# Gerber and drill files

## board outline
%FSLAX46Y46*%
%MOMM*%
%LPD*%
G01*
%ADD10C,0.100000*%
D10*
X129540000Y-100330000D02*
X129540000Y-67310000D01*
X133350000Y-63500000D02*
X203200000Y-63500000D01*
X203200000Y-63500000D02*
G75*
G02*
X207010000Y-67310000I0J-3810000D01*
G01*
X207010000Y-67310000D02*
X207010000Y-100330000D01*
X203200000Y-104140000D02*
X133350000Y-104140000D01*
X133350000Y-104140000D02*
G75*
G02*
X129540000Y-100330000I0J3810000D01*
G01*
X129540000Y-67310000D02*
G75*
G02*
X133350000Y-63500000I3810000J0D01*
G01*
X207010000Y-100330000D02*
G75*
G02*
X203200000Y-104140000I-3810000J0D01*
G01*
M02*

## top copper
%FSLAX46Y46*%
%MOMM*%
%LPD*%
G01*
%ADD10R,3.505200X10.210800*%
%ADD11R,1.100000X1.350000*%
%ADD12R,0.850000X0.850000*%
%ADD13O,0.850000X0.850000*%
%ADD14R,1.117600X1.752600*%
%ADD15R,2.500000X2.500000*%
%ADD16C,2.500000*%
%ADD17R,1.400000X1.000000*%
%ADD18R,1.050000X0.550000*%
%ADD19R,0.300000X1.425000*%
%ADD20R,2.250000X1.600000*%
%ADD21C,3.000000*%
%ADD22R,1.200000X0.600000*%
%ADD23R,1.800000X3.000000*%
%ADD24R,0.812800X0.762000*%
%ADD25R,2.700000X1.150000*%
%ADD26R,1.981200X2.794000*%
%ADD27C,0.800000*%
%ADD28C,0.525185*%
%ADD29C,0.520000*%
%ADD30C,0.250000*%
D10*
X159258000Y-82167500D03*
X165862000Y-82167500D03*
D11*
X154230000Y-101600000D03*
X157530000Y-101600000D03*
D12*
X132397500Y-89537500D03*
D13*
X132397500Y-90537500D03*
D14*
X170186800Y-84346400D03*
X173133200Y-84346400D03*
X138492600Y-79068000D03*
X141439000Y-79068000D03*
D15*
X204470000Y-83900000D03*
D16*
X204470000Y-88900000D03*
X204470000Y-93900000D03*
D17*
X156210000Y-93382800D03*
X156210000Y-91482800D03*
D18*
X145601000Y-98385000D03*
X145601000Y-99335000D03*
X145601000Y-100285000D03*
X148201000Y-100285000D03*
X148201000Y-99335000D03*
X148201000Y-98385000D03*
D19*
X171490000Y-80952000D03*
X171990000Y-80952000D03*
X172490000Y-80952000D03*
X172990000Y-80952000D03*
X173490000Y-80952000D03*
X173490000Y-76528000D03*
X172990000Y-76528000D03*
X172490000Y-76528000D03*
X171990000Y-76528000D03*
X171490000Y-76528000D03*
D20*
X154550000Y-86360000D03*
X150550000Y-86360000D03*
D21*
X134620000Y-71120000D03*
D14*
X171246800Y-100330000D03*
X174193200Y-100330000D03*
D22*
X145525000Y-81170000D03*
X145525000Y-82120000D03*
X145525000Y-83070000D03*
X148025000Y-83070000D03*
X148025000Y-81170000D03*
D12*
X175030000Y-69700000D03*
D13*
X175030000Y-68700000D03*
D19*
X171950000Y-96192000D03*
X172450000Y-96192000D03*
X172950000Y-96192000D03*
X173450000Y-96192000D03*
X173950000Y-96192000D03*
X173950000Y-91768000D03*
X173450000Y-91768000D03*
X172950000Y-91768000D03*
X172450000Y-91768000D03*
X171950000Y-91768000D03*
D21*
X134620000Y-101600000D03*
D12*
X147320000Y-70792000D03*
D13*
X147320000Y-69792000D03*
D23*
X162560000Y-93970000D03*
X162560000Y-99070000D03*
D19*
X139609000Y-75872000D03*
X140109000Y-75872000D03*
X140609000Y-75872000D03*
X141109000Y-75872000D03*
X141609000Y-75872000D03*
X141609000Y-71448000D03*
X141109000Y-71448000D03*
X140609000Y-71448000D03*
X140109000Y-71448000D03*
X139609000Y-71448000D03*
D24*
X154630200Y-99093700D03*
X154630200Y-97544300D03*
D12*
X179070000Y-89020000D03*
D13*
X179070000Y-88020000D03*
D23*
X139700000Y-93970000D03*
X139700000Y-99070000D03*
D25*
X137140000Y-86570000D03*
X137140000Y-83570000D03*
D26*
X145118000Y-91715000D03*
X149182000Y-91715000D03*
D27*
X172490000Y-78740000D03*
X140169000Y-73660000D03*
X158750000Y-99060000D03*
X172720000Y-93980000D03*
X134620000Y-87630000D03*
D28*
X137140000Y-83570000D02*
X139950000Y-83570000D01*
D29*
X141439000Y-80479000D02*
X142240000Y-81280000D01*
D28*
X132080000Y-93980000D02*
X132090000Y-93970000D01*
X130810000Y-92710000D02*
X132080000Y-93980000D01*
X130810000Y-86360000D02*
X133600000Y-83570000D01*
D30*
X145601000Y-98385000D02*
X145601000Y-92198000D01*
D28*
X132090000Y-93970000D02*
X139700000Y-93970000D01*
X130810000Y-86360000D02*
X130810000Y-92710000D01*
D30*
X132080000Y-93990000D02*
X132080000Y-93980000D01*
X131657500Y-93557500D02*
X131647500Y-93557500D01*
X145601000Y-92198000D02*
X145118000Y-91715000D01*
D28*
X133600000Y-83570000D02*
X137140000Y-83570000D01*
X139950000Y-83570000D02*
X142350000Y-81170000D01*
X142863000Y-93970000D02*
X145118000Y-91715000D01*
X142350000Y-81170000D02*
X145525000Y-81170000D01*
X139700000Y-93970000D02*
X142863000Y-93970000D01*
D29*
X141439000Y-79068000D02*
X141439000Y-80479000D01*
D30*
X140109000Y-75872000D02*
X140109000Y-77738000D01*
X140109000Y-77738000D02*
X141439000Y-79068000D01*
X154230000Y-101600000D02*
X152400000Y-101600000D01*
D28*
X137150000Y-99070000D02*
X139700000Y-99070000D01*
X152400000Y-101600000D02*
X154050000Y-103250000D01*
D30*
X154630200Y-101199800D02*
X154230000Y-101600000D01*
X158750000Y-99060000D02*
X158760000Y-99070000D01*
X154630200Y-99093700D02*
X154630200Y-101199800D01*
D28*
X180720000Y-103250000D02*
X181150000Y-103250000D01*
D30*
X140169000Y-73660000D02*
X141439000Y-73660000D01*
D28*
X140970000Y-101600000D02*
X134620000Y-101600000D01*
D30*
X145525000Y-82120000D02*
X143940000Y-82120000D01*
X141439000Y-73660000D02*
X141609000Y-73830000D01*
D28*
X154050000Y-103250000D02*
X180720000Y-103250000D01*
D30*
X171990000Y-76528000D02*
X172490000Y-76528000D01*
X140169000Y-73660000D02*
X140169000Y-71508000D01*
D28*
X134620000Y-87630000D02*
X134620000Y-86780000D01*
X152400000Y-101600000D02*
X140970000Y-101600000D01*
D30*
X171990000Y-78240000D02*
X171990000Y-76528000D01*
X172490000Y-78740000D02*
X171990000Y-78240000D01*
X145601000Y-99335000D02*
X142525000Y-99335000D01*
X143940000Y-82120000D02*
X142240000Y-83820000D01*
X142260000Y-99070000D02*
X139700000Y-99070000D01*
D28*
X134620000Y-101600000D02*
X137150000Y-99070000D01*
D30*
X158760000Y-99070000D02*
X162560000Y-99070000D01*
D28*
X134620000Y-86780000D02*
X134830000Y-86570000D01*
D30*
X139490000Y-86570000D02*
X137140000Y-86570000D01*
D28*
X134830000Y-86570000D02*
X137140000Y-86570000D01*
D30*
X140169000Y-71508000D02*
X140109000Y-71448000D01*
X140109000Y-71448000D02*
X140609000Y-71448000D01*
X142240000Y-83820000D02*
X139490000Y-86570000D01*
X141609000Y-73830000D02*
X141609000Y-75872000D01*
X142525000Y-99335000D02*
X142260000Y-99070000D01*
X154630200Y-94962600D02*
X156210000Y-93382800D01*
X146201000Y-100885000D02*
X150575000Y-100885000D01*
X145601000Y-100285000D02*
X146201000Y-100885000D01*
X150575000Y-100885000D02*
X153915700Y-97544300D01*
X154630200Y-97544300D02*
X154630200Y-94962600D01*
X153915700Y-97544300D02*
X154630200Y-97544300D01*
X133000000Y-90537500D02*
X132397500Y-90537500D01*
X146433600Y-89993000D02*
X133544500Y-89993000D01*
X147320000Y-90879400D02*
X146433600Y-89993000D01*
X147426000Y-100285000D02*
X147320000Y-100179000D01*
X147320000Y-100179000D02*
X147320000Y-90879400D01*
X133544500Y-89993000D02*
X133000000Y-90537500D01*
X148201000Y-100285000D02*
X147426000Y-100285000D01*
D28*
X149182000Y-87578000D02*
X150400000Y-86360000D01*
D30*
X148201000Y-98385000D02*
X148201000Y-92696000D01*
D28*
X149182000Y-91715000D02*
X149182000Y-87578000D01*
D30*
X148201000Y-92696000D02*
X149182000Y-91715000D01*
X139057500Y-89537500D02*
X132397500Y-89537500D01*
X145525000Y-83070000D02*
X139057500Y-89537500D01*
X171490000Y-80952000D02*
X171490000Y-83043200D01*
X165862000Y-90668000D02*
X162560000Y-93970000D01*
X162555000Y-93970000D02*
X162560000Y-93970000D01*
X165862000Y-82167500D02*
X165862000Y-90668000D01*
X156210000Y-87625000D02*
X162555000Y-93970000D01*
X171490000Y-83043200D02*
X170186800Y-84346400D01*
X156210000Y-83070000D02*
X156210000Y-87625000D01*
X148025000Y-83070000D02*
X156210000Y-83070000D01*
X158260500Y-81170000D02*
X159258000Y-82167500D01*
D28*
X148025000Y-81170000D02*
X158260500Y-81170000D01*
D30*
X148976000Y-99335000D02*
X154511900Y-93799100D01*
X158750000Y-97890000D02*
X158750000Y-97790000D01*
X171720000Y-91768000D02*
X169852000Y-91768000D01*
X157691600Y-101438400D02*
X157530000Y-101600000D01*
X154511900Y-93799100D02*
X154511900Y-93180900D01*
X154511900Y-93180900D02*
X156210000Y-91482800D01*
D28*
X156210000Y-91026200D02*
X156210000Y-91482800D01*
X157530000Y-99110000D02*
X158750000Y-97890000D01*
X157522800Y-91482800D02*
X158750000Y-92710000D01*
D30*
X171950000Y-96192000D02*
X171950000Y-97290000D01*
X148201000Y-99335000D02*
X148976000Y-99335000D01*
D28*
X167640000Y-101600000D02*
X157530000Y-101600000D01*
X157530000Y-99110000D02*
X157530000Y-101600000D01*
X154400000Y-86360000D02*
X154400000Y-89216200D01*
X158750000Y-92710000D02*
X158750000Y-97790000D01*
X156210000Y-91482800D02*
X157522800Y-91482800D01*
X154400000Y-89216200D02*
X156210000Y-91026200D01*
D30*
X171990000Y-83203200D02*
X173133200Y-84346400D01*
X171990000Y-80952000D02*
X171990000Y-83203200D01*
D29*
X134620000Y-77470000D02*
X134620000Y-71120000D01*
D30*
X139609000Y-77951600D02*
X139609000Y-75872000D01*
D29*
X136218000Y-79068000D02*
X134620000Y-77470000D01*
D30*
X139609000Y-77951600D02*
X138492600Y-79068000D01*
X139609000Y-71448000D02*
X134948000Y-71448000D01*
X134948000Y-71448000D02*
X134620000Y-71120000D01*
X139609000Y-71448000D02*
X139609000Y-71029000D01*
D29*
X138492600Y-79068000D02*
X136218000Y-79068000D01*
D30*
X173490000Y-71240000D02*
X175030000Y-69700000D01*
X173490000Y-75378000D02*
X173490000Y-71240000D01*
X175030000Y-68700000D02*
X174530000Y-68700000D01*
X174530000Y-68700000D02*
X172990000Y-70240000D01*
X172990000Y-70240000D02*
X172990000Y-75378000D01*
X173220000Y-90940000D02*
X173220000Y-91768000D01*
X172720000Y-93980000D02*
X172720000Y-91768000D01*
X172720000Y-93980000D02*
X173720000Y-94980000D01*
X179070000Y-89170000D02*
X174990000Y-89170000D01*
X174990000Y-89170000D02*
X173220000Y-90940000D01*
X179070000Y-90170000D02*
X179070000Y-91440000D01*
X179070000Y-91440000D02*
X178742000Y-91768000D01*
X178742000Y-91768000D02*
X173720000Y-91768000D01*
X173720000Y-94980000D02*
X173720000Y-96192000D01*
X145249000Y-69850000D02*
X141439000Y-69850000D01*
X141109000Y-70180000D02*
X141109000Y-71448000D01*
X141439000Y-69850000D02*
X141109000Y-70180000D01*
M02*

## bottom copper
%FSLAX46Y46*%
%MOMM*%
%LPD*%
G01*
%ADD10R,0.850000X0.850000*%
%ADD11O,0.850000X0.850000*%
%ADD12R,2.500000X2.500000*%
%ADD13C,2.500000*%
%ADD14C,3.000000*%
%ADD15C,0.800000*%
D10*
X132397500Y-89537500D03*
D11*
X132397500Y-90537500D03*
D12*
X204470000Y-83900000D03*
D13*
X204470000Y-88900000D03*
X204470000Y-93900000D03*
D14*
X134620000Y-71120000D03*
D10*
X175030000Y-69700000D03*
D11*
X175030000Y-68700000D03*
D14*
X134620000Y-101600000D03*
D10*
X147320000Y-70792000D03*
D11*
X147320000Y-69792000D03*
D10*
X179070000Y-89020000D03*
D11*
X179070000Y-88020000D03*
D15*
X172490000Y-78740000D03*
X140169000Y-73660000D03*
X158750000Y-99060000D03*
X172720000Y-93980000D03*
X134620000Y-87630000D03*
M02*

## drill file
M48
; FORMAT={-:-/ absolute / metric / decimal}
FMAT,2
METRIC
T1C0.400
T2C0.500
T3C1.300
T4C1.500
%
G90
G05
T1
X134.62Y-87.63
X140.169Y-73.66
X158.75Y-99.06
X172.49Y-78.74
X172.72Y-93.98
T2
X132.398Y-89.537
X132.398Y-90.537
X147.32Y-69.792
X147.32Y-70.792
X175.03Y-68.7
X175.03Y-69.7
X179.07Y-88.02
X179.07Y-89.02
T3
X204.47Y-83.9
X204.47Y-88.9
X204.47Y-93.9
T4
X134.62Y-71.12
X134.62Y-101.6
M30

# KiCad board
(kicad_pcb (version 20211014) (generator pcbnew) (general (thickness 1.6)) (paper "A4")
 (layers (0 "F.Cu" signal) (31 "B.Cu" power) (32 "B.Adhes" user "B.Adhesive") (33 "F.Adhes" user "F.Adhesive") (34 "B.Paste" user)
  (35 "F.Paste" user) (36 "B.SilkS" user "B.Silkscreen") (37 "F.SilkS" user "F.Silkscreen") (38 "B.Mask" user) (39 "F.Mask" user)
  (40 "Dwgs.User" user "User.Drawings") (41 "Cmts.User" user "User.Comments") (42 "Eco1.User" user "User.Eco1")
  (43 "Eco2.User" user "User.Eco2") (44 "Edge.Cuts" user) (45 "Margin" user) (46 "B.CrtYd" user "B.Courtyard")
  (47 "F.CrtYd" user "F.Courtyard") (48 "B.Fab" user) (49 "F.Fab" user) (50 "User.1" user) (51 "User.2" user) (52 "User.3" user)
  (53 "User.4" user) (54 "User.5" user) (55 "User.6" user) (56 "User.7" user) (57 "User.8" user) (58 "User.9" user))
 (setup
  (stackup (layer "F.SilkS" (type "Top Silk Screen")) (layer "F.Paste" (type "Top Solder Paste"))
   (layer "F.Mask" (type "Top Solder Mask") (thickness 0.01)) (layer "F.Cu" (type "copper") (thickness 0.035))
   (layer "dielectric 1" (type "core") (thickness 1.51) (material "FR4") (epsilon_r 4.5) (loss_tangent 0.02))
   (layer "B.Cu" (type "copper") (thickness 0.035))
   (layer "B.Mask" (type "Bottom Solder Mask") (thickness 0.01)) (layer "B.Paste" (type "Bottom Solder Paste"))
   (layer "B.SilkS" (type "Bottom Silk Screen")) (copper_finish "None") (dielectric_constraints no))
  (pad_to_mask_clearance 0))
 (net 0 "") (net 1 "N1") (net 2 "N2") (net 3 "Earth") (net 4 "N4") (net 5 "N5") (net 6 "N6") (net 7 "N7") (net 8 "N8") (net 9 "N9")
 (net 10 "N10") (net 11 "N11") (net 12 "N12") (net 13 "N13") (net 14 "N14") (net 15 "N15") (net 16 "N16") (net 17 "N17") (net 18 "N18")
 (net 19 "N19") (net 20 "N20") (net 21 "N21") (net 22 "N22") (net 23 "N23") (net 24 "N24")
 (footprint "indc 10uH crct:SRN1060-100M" (layer "F.Cu") (at 162.56 82.1675)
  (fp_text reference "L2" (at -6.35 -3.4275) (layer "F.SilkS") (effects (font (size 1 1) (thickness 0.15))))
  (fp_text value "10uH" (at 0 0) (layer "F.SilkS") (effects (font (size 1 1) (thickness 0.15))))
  (pad "1" smd rect (at -3.302 0) (size 3.5052 10.2108) (layers "F.Cu" "F.Paste" "F.Mask") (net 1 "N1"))
  (pad "2" smd rect (at 3.302 0) (size 3.5052 10.2108) (layers "F.Cu" "F.Paste" "F.Mask") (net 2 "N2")))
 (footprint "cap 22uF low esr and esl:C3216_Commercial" (layer "F.Cu") (at 155.88 101.6)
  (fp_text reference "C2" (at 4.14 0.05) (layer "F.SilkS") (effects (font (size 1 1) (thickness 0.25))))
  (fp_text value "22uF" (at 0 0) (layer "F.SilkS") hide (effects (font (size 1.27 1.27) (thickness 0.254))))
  (pad "1" smd rect (at -1.65 0) (size 1.1 1.35) (layers "F.Cu" "F.Paste" "F.Mask") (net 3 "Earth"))
  (pad "2" smd rect (at 1.65 0) (size 1.1 1.35) (layers "F.Cu" "F.Paste" "F.Mask") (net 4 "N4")))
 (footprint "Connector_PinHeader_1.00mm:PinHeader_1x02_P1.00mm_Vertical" (layer "F.Cu") (at 132.3975 89.5375)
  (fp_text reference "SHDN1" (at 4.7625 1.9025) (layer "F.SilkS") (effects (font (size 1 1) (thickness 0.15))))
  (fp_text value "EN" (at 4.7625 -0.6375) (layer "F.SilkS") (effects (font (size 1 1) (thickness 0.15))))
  (pad "1" thru_hole rect (at 0 0) (size 0.85 0.85) (drill 0.5) (layers *.Cu *.Mask) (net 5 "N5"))
  (pad "2" thru_hole oval (at 0 1) (size 0.85 0.85) (drill 0.5) (layers *.Cu *.Mask) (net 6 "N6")))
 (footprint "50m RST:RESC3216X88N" (layer "F.Cu") (at 171.66 84.3464)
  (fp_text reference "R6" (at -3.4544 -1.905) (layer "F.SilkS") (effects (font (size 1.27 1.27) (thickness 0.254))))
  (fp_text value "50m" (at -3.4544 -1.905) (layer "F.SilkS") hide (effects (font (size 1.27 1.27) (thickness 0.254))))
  (pad "1" smd rect (at -1.4732 0) (size 1.1176 1.7526) (layers "F.Cu" "F.Paste" "F.Mask") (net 2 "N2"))
  (pad "2" smd rect (at 1.4732 0) (size 1.1176 1.7526) (layers "F.Cu" "F.Paste" "F.Mask") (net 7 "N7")))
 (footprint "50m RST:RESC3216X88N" (layer "F.Cu") (at 139.9658 79.068)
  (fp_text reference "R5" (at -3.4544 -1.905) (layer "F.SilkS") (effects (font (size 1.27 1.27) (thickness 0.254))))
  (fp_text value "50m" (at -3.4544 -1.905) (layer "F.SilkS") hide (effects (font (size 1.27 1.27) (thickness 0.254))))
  (pad "1" smd rect (at -1.4732 0) (size 1.1176 1.7526) (layers "F.Cu" "F.Paste" "F.Mask") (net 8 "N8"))
  (pad "2" smd rect (at 1.4732 0) (size 1.1176 1.7526) (layers "F.Cu" "F.Paste" "F.Mask") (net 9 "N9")))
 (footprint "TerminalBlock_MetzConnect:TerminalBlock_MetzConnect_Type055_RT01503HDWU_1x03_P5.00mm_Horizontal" (layer "F.Cu")
  (at 204.47 83.9 -90)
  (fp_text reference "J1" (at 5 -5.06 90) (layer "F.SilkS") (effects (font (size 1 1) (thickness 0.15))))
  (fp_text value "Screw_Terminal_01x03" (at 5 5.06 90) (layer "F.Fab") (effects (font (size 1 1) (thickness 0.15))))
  (pad "1" thru_hole rect (at 0 0 270) (size 2.5 2.5) (drill 1.3) (layers *.Cu *.Mask) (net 7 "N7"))
  (pad "2" thru_hole circle (at 5 0 270) (size 2.5 2.5) (drill 1.3) (layers *.Cu *.Mask) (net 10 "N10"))
  (pad "3" thru_hole circle (at 10 0 270) (size 2.5 2.5) (drill 1.3) (layers *.Cu *.Mask) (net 3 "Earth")))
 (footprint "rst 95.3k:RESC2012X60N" (layer "F.Cu") (at 156.21 92.4328 90)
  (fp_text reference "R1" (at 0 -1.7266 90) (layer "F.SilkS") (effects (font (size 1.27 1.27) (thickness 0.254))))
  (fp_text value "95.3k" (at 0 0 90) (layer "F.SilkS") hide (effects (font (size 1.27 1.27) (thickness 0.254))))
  (pad "1" smd rect (at -0.95 0 90) (size 1 1.4) (layers "F.Cu" "F.Paste" "F.Mask") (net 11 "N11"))
  (pad "2" smd rect (at 0.95 0 90) (size 1 1.4) (layers "F.Cu" "F.Paste" "F.Mask") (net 4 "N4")))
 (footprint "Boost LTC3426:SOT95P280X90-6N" (layer "F.Cu") (at 146.901 99.335)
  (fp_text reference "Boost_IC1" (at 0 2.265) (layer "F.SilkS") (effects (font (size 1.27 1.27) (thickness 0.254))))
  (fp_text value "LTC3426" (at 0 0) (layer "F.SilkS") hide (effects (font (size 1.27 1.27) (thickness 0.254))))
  (pad "1" smd rect (at -1.3 -0.95 90) (size 0.55 1.05) (layers "F.Cu" "F.Paste" "F.Mask") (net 9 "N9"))
  (pad "2" smd rect (at -1.3 0 90) (size 0.55 1.05) (layers "F.Cu" "F.Paste" "F.Mask") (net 3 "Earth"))
  (pad "3" smd rect (at -1.3 0.95 90) (size 0.55 1.05) (layers "F.Cu" "F.Paste" "F.Mask") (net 11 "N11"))
  (pad "4" smd rect (at 1.3 0.95 90) (size 0.55 1.05) (layers "F.Cu" "F.Paste" "F.Mask") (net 6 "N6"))
  (pad "5" smd rect (at 1.3 0 90) (size 0.55 1.05) (layers "F.Cu" "F.Paste" "F.Mask") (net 4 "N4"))
  (pad "6" smd rect (at 1.3 -0.95 90) (size 0.55 1.05) (layers "F.Cu" "F.Paste" "F.Mask") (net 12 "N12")))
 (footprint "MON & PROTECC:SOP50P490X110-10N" (layer "F.Cu") (at 172.49 78.74 90)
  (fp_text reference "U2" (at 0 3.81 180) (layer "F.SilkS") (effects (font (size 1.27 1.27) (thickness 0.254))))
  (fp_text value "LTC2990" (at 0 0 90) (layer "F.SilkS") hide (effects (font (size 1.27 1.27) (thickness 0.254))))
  (pad "1" smd rect (at -2.212 -1 180) (size 0.3 1.425) (layers "F.Cu" "F.Paste" "F.Mask") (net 2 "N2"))
  (pad "2" smd rect (at -2.212 -0.5 180) (size 0.3 1.425) (layers "F.Cu" "F.Paste" "F.Mask") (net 7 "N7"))
  (pad "3" smd rect (at -2.212 0 180) (size 0.3 1.425) (layers "F.Cu" "F.Paste" "F.Mask") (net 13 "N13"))
  (pad "4" smd rect (at -2.212 0.5 180) (size 0.3 1.425) (layers "F.Cu" "F.Paste" "F.Mask") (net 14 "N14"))
  (pad "5" smd rect (at -2.212 1 180) (size 0.3 1.425) (layers "F.Cu" "F.Paste" "F.Mask") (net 3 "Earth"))
  (pad "6" smd rect (at 2.212 1 180) (size 0.3 1.425) (layers "F.Cu" "F.Paste" "F.Mask") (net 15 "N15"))
  (pad "7" smd rect (at 2.212 0.5 180) (size 0.3 1.425) (layers "F.Cu" "F.Paste" "F.Mask") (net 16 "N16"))
  (pad "8" smd rect (at 2.212 0 180) (size 0.3 1.425) (layers "F.Cu" "F.Paste" "F.Mask") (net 3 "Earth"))
  (pad "9" smd rect (at 2.212 -0.5 180) (size 0.3 1.425) (layers "F.Cu" "F.Paste" "F.Mask") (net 3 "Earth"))
  (pad "10" smd rect (at 2.212 -1 180) (size 0.3 1.425) (layers "F.Cu" "F.Paste" "F.Mask") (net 2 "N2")))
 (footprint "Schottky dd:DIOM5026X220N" (layer "F.Cu") (at 152.55 86.36 180)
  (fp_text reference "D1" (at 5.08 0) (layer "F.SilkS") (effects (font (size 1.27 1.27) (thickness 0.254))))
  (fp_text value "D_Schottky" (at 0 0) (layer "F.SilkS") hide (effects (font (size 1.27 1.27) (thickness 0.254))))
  (pad "1" smd rect (at -2 0 270) (size 1.6 2.25) (layers "F.Cu" "F.Paste" "F.Mask") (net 4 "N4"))
  (pad "2" smd rect (at 2 0 270) (size 1.6 2.25) (layers "F.Cu" "F.Paste" "F.Mask") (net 12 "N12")))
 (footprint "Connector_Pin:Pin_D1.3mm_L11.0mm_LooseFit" (layer "F.Cu") (at 134.62 71.12)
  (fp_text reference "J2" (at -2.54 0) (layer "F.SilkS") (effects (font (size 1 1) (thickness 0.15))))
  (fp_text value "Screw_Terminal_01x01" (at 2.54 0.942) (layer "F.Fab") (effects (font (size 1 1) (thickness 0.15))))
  (pad "1" thru_hole circle (at 0 0) (size 3 3) (drill 1.5) (layers *.Cu *.Mask) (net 8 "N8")))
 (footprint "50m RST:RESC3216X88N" (layer "F.Cu") (at 172.72 100.33)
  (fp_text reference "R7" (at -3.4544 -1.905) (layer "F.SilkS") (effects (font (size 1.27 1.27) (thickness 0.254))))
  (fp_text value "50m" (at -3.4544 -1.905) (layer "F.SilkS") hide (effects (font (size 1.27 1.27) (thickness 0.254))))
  (pad "1" smd rect (at -1.4732 0) (size 1.1176 1.7526) (layers "F.Cu" "F.Paste" "F.Mask") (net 4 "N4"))
  (pad "2" smd rect (at 1.4732 0) (size 1.1176 1.7526) (layers "F.Cu" "F.Paste" "F.Mask") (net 10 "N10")))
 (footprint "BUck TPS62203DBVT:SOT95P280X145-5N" (layer "F.Cu") (at 146.775 82.12)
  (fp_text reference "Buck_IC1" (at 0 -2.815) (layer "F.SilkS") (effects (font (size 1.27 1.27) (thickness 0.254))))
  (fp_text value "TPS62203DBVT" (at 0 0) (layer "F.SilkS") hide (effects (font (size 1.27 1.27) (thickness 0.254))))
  (pad "1" smd rect (at -1.25 -0.95 90) (size 0.6 1.2) (layers "F.Cu" "F.Paste" "F.Mask") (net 9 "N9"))
  (pad "2" smd rect (at -1.25 0 90) (size 0.6 1.2) (layers "F.Cu" "F.Paste" "F.Mask") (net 3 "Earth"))
  (pad "3" smd rect (at -1.25 0.95 90) (size 0.6 1.2) (layers "F.Cu" "F.Paste" "F.Mask") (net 5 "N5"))
  (pad "4" smd rect (at 1.25 0.95 90) (size 0.6 1.2) (layers "F.Cu" "F.Paste" "F.Mask") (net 2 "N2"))
  (pad "5" smd rect (at 1.25 -0.95 90) (size 0.6 1.2) (layers "F.Cu" "F.Paste" "F.Mask") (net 1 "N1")))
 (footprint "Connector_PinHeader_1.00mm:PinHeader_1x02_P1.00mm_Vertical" (layer "F.Cu") (at 175.03 69.7 180)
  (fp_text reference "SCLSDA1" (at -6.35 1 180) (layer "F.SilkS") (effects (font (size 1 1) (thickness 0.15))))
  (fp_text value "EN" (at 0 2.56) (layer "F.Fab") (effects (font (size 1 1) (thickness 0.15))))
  (pad "1" thru_hole rect (at 0 0 180) (size 0.85 0.85) (drill 0.5) (layers *.Cu *.Mask) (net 15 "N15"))
  (pad "2" thru_hole oval (at 0 1 180) (size 0.85 0.85) (drill 0.5) (layers *.Cu *.Mask) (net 16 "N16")))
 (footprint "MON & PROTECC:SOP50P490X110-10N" (layer "F.Cu") (at 172.95 93.98 90)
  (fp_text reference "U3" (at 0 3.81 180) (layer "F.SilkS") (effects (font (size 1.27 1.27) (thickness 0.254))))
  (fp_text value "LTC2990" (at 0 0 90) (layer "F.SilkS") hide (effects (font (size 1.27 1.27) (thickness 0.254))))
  (pad "1" smd rect (at -2.212 -1 180) (size 0.3 1.425) (layers "F.Cu" "F.Paste" "F.Mask") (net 4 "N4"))
  (pad "2" smd rect (at -2.212 -0.5 180) (size 0.3 1.425) (layers "F.Cu" "F.Paste" "F.Mask") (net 10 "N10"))
  (pad "3" smd rect (at -2.212 0 180) (size 0.3 1.425) (layers "F.Cu" "F.Paste" "F.Mask") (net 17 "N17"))
  (pad "4" smd rect (at -2.212 0.5 180) (size 0.3 1.425) (layers "F.Cu" "F.Paste" "F.Mask") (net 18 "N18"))
  (pad "5" smd rect (at -2.212 1 180) (size 0.3 1.425) (layers "F.Cu" "F.Paste" "F.Mask") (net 3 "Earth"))
  (pad "6" smd rect (at 2.212 1 180) (size 0.3 1.425) (layers "F.Cu" "F.Paste" "F.Mask") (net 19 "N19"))
  (pad "7" smd rect (at 2.212 0.5 180) (size 0.3 1.425) (layers "F.Cu" "F.Paste" "F.Mask") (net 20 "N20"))
  (pad "8" smd rect (at 2.212 0 180) (size 0.3 1.425) (layers "F.Cu" "F.Paste" "F.Mask") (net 3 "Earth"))
  (pad "9" smd rect (at 2.212 -0.5 180) (size 0.3 1.425) (layers "F.Cu" "F.Paste" "F.Mask") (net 3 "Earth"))
  (pad "10" smd rect (at 2.212 -1 180) (size 0.3 1.425) (layers "F.Cu" "F.Paste" "F.Mask") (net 4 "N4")))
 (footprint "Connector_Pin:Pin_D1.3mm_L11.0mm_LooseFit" (layer "F.Cu") (at 134.62 101.6)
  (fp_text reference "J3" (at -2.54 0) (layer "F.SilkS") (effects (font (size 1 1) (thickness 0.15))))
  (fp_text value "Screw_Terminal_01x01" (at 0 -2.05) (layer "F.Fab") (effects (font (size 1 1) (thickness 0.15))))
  (pad "1" thru_hole circle (at 0 0) (size 3 3) (drill 1.5) (layers *.Cu *.Mask) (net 3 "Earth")))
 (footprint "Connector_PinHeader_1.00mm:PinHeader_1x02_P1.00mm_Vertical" (layer "F.Cu") (at 147.32 70.792 180)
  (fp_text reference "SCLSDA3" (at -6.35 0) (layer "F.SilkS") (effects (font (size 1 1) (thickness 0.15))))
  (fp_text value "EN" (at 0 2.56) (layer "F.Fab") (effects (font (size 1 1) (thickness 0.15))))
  (pad "1" thru_hole rect (at 0 0 180) (size 0.85 0.85) (drill 0.5) (layers *.Cu *.Mask) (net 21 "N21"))
  (pad "2" thru_hole oval (at 0 1 180) (size 0.85 0.85) (drill 0.5) (layers *.Cu *.Mask) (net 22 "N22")))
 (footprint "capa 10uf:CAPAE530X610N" (layer "F.Cu") (at 162.56 96.52 -90)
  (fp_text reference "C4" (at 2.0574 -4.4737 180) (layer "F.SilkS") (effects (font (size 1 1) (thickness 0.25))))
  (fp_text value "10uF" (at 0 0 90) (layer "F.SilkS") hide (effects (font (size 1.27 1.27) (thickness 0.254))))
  (pad "1" smd rect (at -2.55 0) (size 1.8 3) (layers "F.Cu" "F.Paste" "F.Mask") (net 2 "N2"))
  (pad "2" smd rect (at 2.55 0) (size 1.8 3) (layers "F.Cu" "F.Paste" "F.Mask") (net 3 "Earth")))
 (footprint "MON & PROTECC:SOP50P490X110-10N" (layer "F.Cu") (at 140.609 73.66 90)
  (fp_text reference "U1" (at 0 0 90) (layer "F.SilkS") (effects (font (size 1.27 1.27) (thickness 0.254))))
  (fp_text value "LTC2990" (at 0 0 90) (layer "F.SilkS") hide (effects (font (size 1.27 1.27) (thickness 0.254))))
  (pad "1" smd rect (at -2.212 -1 180) (size 0.3 1.425) (layers "F.Cu" "F.Paste" "F.Mask") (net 8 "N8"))
  (pad "2" smd rect (at -2.212 -0.5 180) (size 0.3 1.425) (layers "F.Cu" "F.Paste" "F.Mask") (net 9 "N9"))
  (pad "3" smd rect (at -2.212 0 180) (size 0.3 1.425) (layers "F.Cu" "F.Paste" "F.Mask") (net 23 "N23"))
  (pad "4" smd rect (at -2.212 0.5 180) (size 0.3 1.425) (layers "F.Cu" "F.Paste" "F.Mask") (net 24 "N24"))
  (pad "5" smd rect (at -2.212 1 180) (size 0.3 1.425) (layers "F.Cu" "F.Paste" "F.Mask") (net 3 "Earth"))
  (pad "6" smd rect (at 2.212 1 180) (size 0.3 1.425) (layers "F.Cu" "F.Paste" "F.Mask") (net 21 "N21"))
  (pad "7" smd rect (at 2.212 0.5 180) (size 0.3 1.425) (layers "F.Cu" "F.Paste" "F.Mask") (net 22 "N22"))
  (pad "8" smd rect (at 2.212 0 180) (size 0.3 1.425) (layers "F.Cu" "F.Paste" "F.Mask") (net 3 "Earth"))
  (pad "9" smd rect (at 2.212 -0.5 180) (size 0.3 1.425) (layers "F.Cu" "F.Paste" "F.Mask") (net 3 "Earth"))
  (pad "10" smd rect (at 2.212 -1 180) (size 0.3 1.425) (layers "F.Cu" "F.Paste" "F.Mask") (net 8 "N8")))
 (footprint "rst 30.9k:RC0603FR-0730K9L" (layer "F.Cu") (at 154.6302 98.319 90)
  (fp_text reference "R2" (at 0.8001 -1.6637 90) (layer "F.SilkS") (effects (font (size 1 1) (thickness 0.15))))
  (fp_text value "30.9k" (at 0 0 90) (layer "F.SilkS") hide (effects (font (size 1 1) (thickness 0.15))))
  (pad "1" smd rect (at -0.7747 0 90) (size 0.762 0.8128) (layers "F.Cu" "F.Paste" "F.Mask") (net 3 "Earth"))
  (pad "2" smd rect (at 0.7747 0 90) (size 0.762 0.8128) (layers "F.Cu" "F.Paste" "F.Mask") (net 11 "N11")))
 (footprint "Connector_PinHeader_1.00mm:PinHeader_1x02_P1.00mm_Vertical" (layer "F.Cu") (at 179.07 89.02 180)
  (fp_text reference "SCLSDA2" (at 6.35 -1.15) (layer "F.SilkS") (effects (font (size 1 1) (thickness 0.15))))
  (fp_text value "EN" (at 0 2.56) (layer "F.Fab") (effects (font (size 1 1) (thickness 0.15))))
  (pad "1" thru_hole rect (at 0 0 180) (size 0.85 0.85) (drill 0.5) (layers *.Cu *.Mask) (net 19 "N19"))
  (pad "2" thru_hole oval (at 0 1 180) (size 0.85 0.85) (drill 0.5) (layers *.Cu *.Mask) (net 20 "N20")))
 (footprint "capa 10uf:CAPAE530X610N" (layer "F.Cu") (at 139.7 96.52 -90)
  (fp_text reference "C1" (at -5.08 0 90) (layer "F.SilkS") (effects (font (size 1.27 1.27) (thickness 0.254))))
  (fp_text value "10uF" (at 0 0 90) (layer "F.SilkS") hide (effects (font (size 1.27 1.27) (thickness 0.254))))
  (pad "1" smd rect (at -2.55 0) (size 1.8 3) (layers "F.Cu" "F.Paste" "F.Mask") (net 9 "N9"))
  (pad "2" smd rect (at 2.55 0) (size 1.8 3) (layers "F.Cu" "F.Paste" "F.Mask") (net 3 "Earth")))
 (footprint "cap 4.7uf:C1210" (layer "F.Cu") (at 137.14 85.07 90)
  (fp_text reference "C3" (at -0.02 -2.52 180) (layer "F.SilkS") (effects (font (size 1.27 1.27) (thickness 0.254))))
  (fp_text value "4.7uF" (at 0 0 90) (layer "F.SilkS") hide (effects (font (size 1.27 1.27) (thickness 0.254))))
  (pad "1" smd rect (at -1.5 0 90) (size 1.15 2.7) (layers "F.Cu" "F.Paste" "F.Mask") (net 3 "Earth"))
  (pad "2" smd rect (at 1.5 0 90) (size 1.15 2.7) (layers "F.Cu" "F.Paste" "F.Mask") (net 9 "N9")))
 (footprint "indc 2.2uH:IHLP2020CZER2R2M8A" (layer "F.Cu") (at 147.15 91.715)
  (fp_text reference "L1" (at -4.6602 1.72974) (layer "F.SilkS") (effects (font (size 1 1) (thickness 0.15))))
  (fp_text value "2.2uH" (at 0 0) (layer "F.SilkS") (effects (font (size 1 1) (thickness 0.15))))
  (pad "1" smd rect (at -2.032 0 90) (size 2.794 1.9812) (layers "F.Cu" "F.Paste" "F.Mask") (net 9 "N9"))
  (pad "2" smd rect (at 2.032 0 90) (size 2.794 1.9812) (layers "F.Cu" "F.Paste" "F.Mask") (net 12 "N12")))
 (gr_line (start 129.54 100.33) (end 129.54 67.31) (layer "Edge.Cuts") (width 0.1))
 (gr_line (start 133.35 63.5) (end 203.2 63.5) (layer "Edge.Cuts") (width 0.1))
 (gr_arc (start 203.2 63.5) (mid 205.894077 64.615923) (end 207.01 67.31) (layer "Edge.Cuts") (width 0.1))
 (gr_line (start 207.01 67.31) (end 207.01 100.33) (layer "Edge.Cuts") (width 0.1))
 (gr_line (start 203.2 104.14) (end 133.35 104.14) (layer "Edge.Cuts") (width 0.1))
 (gr_arc (start 133.35 104.14) (mid 130.655923 103.024077) (end 129.54 100.33) (layer "Edge.Cuts") (width 0.1))
 (gr_arc (start 129.54 67.31) (mid 130.655923 64.615923) (end 133.35 63.5) (layer "Edge.Cuts") (width 0.1))
 (gr_arc (start 207.01 100.33) (mid 205.894077 103.024077) (end 203.2 104.14) (layer "Edge.Cuts") (width 0.1))
 (segment (start 137.14 83.57) (end 139.95 83.57) (width 0.525185) (layer "F.Cu") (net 9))
 (segment (start 141.439 80.479) (end 142.24 81.28) (width 0.52) (layer "F.Cu") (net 9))
 (segment (start 132.08 93.98) (end 132.09 93.97) (width 0.525185) (layer "F.Cu") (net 9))
 (segment (start 130.81 92.71) (end 132.08 93.98) (width 0.525185) (layer "F.Cu") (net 9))
 (segment (start 130.81 86.36) (end 133.6 83.57) (width 0.525185) (layer "F.Cu") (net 9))
 (segment (start 145.601 98.385) (end 145.601 92.198) (width 0.25) (layer "F.Cu") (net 9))
 (segment (start 132.09 93.97) (end 139.7 93.97) (width 0.525185) (layer "F.Cu") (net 9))
 (segment (start 130.81 86.36) (end 130.81 92.71) (width 0.525185) (layer "F.Cu") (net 9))
 (segment (start 132.08 93.99) (end 132.08 93.98) (width 0.25) (layer "F.Cu") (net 9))
 (segment (start 131.6575 93.5575) (end 131.6475 93.5575) (width 0.25) (layer "F.Cu") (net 9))
 (segment (start 145.601 92.198) (end 145.118 91.715) (width 0.25) (layer "F.Cu") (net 9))
 (segment (start 133.6 83.57) (end 137.14 83.57) (width 0.525185) (layer "F.Cu") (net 9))
 (segment (start 139.95 83.57) (end 142.35 81.17) (width 0.525185) (layer "F.Cu") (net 9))
 (segment (start 142.863 93.97) (end 145.118 91.715) (width 0.525185) (layer "F.Cu") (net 9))
 (segment (start 142.35 81.17) (end 145.525 81.17) (width 0.525185) (layer "F.Cu") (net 9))
 (segment (start 139.7 93.97) (end 142.863 93.97) (width 0.525185) (layer "F.Cu") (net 9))
 (segment (start 141.439 79.068) (end 141.439 80.479) (width 0.52) (layer "F.Cu") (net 9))
 (segment (start 140.109 75.872) (end 140.109 77.738) (width 0.25) (layer "F.Cu") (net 9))
 (segment (start 140.109 77.738) (end 141.439 79.068) (width 0.25) (layer "F.Cu") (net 9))
 (segment (start 154.23 101.6) (end 152.4 101.6) (width 0.25) (layer "F.Cu") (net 3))
 (segment (start 137.15 99.07) (end 139.7 99.07) (width 0.525185) (layer "F.Cu") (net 3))
 (segment (start 152.4 101.6) (end 154.05 103.25) (width 0.525185) (layer "F.Cu") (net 3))
 (segment (start 154.6302 101.1998) (end 154.23 101.6) (width 0.25) (layer "F.Cu") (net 3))
 (segment (start 158.75 99.06) (end 158.76 99.07) (width 0.25) (layer "F.Cu") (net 3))
 (segment (start 154.6302 99.0937) (end 154.6302 101.1998) (width 0.25) (layer "F.Cu") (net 3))
 (segment (start 180.72 103.25) (end 181.15 103.25) (width 0.525185) (layer "F.Cu") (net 3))
 (segment (start 140.169 73.66) (end 141.439 73.66) (width 0.25) (layer "F.Cu") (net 3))
 (segment (start 140.97 101.6) (end 134.62 101.6) (width 0.525185) (layer "F.Cu") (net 3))
 (segment (start 145.525 82.12) (end 143.94 82.12) (width 0.25) (layer "F.Cu") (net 3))
 (segment (start 141.439 73.66) (end 141.609 73.83) (width 0.25) (layer "F.Cu") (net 3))
 (segment (start 154.05 103.25) (end 180.72 103.25) (width 0.525185) (layer "F.Cu") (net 3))
 (segment (start 171.99 76.528) (end 172.49 76.528) (width 0.25) (layer "F.Cu") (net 3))
 (segment (start 140.169 73.66) (end 140.169 71.508) (width 0.25) (layer "F.Cu") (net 3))
 (segment (start 134.62 87.63) (end 134.62 86.78) (width 0.525185) (layer "F.Cu") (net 3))
 (segment (start 152.4 101.6) (end 140.97 101.6) (width 0.525185) (layer "F.Cu") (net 3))
 (segment (start 171.99 78.24) (end 171.99 76.528) (width 0.25) (layer "F.Cu") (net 3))
 (segment (start 172.49 78.74) (end 171.99 78.24) (width 0.25) (layer "F.Cu") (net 3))
 (segment (start 145.601 99.335) (end 142.525 99.335) (width 0.25) (layer "F.Cu") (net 3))
 (segment (start 143.94 82.12) (end 142.24 83.82) (width 0.25) (layer "F.Cu") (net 3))
 (segment (start 142.26 99.07) (end 139.7 99.07) (width 0.25) (layer "F.Cu") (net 3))
 (segment (start 134.62 101.6) (end 137.15 99.07) (width 0.525185) (layer "F.Cu") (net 3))
 (segment (start 158.76 99.07) (end 162.56 99.07) (width 0.25) (layer "F.Cu") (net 3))
 (segment (start 134.62 86.78) (end 134.83 86.57) (width 0.525185) (layer "F.Cu") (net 3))
 (segment (start 139.49 86.57) (end 137.14 86.57) (width 0.25) (layer "F.Cu") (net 3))
 (segment (start 134.83 86.57) (end 137.14 86.57) (width 0.525185) (layer "F.Cu") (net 3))
 (segment (start 140.169 71.508) (end 140.109 71.448) (width 0.25) (layer "F.Cu") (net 3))
 (segment (start 140.109 71.448) (end 140.609 71.448) (width 0.25) (layer "F.Cu") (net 3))
 (segment (start 142.24 83.82) (end 139.49 86.57) (width 0.25) (layer "F.Cu") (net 3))
 (segment (start 141.609 73.83) (end 141.609 75.872) (width 0.25) (layer "F.Cu") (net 3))
 (segment (start 142.525 99.335) (end 142.26 99.07) (width 0.25) (layer "F.Cu") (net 3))
 (via (at 172.49 78.74) (size 0.8) (drill 0.4) (layers "F.Cu" "B.Cu") (free) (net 3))
 (via (at 140.169 73.66) (size 0.8) (drill 0.4) (layers "F.Cu" "B.Cu") (free) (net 3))
 (via (at 158.75 99.06) (size 0.8) (drill 0.4) (layers "F.Cu" "B.Cu") (free) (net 3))
 (via (at 172.72 93.98) (size 0.8) (drill 0.4) (layers "F.Cu" "B.Cu") (free) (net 3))
 (via (at 134.62 87.63) (size 0.8) (drill 0.4) (layers "F.Cu" "B.Cu") (free) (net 3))
 (segment (start 154.6302 94.9626) (end 156.21 93.3828) (width 0.25) (layer "F.Cu") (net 11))
 (segment (start 146.201 100.885) (end 150.575 100.885) (width 0.25) (layer "F.Cu") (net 11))
 (segment (start 145.601 100.285) (end 146.201 100.885) (width 0.25) (layer "F.Cu") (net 11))
 (segment (start 150.575 100.885) (end 153.9157 97.5443) (width 0.25) (layer "F.Cu") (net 11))
 (segment (start 154.6302 97.5443) (end 154.6302 94.9626) (width 0.25) (layer "F.Cu") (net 11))
 (segment (start 153.9157 97.5443) (end 154.6302 97.5443) (width 0.25) (layer "F.Cu") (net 11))
 (segment (start 133 90.5375) (end 132.3975 90.5375) (width 0.25) (layer "F.Cu") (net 6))
 (segment (start 146.4336 89.993) (end 133.5445 89.993) (width 0.25) (layer "F.Cu") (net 6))
 (segment (start 147.32 90.8794) (end 146.4336 89.993) (width 0.25) (layer "F.Cu") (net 6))
 (segment (start 147.426 100.285) (end 147.32 100.179) (width 0.25) (layer "F.Cu") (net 6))
 (segment (start 147.32 100.179) (end 147.32 90.8794) (width 0.25) (layer "F.Cu") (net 6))
 (segment (start 133.5445 89.993) (end 133 90.5375) (width 0.25) (layer "F.Cu") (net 6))
 (segment (start 148.201 100.285) (end 147.426 100.285) (width 0.25) (layer "F.Cu") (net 6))
 (segment (start 149.182 87.578) (end 150.4 86.36) (width 0.525185) (layer "F.Cu") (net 12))
 (segment (start 148.201 98.385) (end 148.201 92.696) (width 0.25) (layer "F.Cu") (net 12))
 (segment (start 149.182 91.715) (end 149.182 87.578) (width 0.525185) (layer "F.Cu") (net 12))
 (segment (start 148.201 92.696) (end 149.182 91.715) (width 0.25) (layer "F.Cu") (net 12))
 (segment (start 139.0575 89.5375) (end 132.3975 89.5375) (width 0.25) (layer "F.Cu") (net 5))
 (segment (start 145.525 83.07) (end 139.0575 89.5375) (width 0.25) (layer "F.Cu") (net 5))
 (segment (start 171.49 80.952) (end 171.49 83.0432) (width 0.25) (layer "F.Cu") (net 2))
 (segment (start 165.862 90.668) (end 162.56 93.97) (width 0.25) (layer "F.Cu") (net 2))
 (segment (start 162.555 93.97) (end 162.56 93.97) (width 0.25) (layer "F.Cu") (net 2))
 (segment (start 165.862 82.1675) (end 165.862 90.668) (width 0.25) (layer "F.Cu") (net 2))
 (segment (start 156.21 87.625) (end 162.555 93.97) (width 0.25) (layer "F.Cu") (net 2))
 (segment (start 171.49 83.0432) (end 170.1868 84.3464) (width 0.25) (layer "F.Cu") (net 2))
 (segment (start 156.21 83.07) (end 156.21 87.625) (width 0.25) (layer "F.Cu") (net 2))
 (segment (start 148.025 83.07) (end 156.21 83.07) (width 0.25) (layer "F.Cu") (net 2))
 (segment (start 158.2605 81.17) (end 159.258 82.1675) (width 0.25) (layer "F.Cu") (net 1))
 (segment (start 148.025 81.17) (end 158.2605 81.17) (width 0.525185) (layer "F.Cu") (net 1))
 (segment (start 148.976 99.335) (end 154.5119 93.7991) (width 0.25) (layer "F.Cu") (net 4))
 (segment (start 158.75 97.89) (end 158.75 97.79) (width 0.25) (layer "F.Cu") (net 4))
 (segment (start 171.72 91.768) (end 169.852 91.768) (width 0.25) (layer "F.Cu") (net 4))
 (segment (start 157.6916 101.4384) (end 157.53 101.6) (width 0.25) (layer "F.Cu") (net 4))
 (segment (start 154.5119 93.7991) (end 154.5119 93.1809) (width 0.25) (layer "F.Cu") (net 4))
 (segment (start 154.5119 93.1809) (end 156.21 91.4828) (width 0.25) (layer "F.Cu") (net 4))
 (segment (start 156.21 91.0262) (end 156.21 91.4828) (width 0.525185) (layer "F.Cu") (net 4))
 (segment (start 157.53 99.11) (end 158.75 97.89) (width 0.525185) (layer "F.Cu") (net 4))
 (segment (start 157.5228 91.4828) (end 158.75 92.71) (width 0.525185) (layer "F.Cu") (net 4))
 (segment (start 171.95 96.192) (end 171.95 97.29) (width 0.25) (layer "F.Cu") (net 4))
 (segment (start 148.201 99.335) (end 148.976 99.335) (width 0.25) (layer "F.Cu") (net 4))
 (segment (start 167.64 101.6) (end 157.53 101.6) (width 0.525185) (layer "F.Cu") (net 4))
 (segment (start 157.53 99.11) (end 157.53 101.6) (width 0.525185) (layer "F.Cu") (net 4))
 (segment (start 154.4 86.36) (end 154.4 89.2162) (width 0.525185) (layer "F.Cu") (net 4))
 (segment (start 158.75 92.71) (end 158.75 97.79) (width 0.525185) (layer "F.Cu") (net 4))
 (segment (start 156.21 91.4828) (end 157.5228 91.4828) (width 0.525185) (layer "F.Cu") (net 4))
 (segment (start 154.4 89.2162) (end 156.21 91.0262) (width 0.525185) (layer "F.Cu") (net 4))
 (segment (start 171.99 83.2032) (end 173.1332 84.3464) (width 0.25) (layer "F.Cu") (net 7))
 (segment (start 171.99 80.952) (end 171.99 83.2032) (width 0.25) (layer "F.Cu") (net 7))
 (segment (start 134.62 77.47) (end 134.62 71.12) (width 0.52) (layer "F.Cu") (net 8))
 (segment (start 139.609 77.9516) (end 139.609 75.872) (width 0.25) (layer "F.Cu") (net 8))
 (segment (start 136.218 79.068) (end 134.62 77.47) (width 0.52) (layer "F.Cu") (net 8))
 (segment (start 139.609 77.9516) (end 138.4926 79.068) (width 0.25) (layer "F.Cu") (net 8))
 (segment (start 139.609 71.448) (end 134.948 71.448) (width 0.25) (layer "F.Cu") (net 8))
 (segment (start 134.948 71.448) (end 134.62 71.12) (width 0.25) (layer "F.Cu") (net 8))
 (segment (start 139.609 71.448) (end 139.609 71.029) (width 0.25) (layer "F.Cu") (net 8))
 (segment (start 138.4926 79.068) (end 136.218 79.068) (width 0.52) (layer "F.Cu") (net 8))
 (segment (start 173.49 71.24) (end 175.03 69.7) (width 0.25) (layer "F.Cu") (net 15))
 (segment (start 173.49 75.378) (end 173.49 71.24) (width 0.25) (layer "F.Cu") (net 15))
 (segment (start 175.03 68.7) (end 174.53 68.7) (width 0.25) (layer "F.Cu") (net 16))
 (segment (start 174.53 68.7) (end 172.99 70.24) (width 0.25) (layer "F.Cu") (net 16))
 (segment (start 172.99 70.24) (end 172.99 75.378) (width 0.25) (layer "F.Cu") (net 16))
 (segment (start 173.22 90.94) (end 173.22 91.768) (width 0.25) (layer "F.Cu") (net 19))
 (segment (start 172.72 93.98) (end 172.72 91.768) (width 0.25) (layer "F.Cu") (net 19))
 (segment (start 172.72 93.98) (end 173.72 94.98) (width 0.25) (layer "F.Cu") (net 19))
 (segment (start 179.07 89.17) (end 174.99 89.17) (width 0.25) (layer "F.Cu") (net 19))
 (segment (start 174.99 89.17) (end 173.22 90.94) (width 0.25) (layer "F.Cu") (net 19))
 (segment (start 179.07 90.17) (end 179.07 91.44) (width 0.25) (layer "F.Cu") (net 19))
 (segment (start 179.07 91.44) (end 178.742 91.768) (width 0.25) (layer "F.Cu") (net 19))
 (segment (start 178.742 91.768) (end 173.72 91.768) (width 0.25) (layer "F.Cu") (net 19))
 (segment (start 173.72 94.98) (end 173.72 96.192) (width 0.25) (layer "F.Cu") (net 19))
 (segment (start 145.249 69.85) (end 141.439 69.85) (width 0.25) (layer "F.Cu") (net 22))
 (segment (start 141.109 70.18) (end 141.109 71.448) (width 0.25) (layer "F.Cu") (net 22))
 (segment (start 141.439 69.85) (end 141.109 70.18) (width 0.25) (layer "F.Cu") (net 22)))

